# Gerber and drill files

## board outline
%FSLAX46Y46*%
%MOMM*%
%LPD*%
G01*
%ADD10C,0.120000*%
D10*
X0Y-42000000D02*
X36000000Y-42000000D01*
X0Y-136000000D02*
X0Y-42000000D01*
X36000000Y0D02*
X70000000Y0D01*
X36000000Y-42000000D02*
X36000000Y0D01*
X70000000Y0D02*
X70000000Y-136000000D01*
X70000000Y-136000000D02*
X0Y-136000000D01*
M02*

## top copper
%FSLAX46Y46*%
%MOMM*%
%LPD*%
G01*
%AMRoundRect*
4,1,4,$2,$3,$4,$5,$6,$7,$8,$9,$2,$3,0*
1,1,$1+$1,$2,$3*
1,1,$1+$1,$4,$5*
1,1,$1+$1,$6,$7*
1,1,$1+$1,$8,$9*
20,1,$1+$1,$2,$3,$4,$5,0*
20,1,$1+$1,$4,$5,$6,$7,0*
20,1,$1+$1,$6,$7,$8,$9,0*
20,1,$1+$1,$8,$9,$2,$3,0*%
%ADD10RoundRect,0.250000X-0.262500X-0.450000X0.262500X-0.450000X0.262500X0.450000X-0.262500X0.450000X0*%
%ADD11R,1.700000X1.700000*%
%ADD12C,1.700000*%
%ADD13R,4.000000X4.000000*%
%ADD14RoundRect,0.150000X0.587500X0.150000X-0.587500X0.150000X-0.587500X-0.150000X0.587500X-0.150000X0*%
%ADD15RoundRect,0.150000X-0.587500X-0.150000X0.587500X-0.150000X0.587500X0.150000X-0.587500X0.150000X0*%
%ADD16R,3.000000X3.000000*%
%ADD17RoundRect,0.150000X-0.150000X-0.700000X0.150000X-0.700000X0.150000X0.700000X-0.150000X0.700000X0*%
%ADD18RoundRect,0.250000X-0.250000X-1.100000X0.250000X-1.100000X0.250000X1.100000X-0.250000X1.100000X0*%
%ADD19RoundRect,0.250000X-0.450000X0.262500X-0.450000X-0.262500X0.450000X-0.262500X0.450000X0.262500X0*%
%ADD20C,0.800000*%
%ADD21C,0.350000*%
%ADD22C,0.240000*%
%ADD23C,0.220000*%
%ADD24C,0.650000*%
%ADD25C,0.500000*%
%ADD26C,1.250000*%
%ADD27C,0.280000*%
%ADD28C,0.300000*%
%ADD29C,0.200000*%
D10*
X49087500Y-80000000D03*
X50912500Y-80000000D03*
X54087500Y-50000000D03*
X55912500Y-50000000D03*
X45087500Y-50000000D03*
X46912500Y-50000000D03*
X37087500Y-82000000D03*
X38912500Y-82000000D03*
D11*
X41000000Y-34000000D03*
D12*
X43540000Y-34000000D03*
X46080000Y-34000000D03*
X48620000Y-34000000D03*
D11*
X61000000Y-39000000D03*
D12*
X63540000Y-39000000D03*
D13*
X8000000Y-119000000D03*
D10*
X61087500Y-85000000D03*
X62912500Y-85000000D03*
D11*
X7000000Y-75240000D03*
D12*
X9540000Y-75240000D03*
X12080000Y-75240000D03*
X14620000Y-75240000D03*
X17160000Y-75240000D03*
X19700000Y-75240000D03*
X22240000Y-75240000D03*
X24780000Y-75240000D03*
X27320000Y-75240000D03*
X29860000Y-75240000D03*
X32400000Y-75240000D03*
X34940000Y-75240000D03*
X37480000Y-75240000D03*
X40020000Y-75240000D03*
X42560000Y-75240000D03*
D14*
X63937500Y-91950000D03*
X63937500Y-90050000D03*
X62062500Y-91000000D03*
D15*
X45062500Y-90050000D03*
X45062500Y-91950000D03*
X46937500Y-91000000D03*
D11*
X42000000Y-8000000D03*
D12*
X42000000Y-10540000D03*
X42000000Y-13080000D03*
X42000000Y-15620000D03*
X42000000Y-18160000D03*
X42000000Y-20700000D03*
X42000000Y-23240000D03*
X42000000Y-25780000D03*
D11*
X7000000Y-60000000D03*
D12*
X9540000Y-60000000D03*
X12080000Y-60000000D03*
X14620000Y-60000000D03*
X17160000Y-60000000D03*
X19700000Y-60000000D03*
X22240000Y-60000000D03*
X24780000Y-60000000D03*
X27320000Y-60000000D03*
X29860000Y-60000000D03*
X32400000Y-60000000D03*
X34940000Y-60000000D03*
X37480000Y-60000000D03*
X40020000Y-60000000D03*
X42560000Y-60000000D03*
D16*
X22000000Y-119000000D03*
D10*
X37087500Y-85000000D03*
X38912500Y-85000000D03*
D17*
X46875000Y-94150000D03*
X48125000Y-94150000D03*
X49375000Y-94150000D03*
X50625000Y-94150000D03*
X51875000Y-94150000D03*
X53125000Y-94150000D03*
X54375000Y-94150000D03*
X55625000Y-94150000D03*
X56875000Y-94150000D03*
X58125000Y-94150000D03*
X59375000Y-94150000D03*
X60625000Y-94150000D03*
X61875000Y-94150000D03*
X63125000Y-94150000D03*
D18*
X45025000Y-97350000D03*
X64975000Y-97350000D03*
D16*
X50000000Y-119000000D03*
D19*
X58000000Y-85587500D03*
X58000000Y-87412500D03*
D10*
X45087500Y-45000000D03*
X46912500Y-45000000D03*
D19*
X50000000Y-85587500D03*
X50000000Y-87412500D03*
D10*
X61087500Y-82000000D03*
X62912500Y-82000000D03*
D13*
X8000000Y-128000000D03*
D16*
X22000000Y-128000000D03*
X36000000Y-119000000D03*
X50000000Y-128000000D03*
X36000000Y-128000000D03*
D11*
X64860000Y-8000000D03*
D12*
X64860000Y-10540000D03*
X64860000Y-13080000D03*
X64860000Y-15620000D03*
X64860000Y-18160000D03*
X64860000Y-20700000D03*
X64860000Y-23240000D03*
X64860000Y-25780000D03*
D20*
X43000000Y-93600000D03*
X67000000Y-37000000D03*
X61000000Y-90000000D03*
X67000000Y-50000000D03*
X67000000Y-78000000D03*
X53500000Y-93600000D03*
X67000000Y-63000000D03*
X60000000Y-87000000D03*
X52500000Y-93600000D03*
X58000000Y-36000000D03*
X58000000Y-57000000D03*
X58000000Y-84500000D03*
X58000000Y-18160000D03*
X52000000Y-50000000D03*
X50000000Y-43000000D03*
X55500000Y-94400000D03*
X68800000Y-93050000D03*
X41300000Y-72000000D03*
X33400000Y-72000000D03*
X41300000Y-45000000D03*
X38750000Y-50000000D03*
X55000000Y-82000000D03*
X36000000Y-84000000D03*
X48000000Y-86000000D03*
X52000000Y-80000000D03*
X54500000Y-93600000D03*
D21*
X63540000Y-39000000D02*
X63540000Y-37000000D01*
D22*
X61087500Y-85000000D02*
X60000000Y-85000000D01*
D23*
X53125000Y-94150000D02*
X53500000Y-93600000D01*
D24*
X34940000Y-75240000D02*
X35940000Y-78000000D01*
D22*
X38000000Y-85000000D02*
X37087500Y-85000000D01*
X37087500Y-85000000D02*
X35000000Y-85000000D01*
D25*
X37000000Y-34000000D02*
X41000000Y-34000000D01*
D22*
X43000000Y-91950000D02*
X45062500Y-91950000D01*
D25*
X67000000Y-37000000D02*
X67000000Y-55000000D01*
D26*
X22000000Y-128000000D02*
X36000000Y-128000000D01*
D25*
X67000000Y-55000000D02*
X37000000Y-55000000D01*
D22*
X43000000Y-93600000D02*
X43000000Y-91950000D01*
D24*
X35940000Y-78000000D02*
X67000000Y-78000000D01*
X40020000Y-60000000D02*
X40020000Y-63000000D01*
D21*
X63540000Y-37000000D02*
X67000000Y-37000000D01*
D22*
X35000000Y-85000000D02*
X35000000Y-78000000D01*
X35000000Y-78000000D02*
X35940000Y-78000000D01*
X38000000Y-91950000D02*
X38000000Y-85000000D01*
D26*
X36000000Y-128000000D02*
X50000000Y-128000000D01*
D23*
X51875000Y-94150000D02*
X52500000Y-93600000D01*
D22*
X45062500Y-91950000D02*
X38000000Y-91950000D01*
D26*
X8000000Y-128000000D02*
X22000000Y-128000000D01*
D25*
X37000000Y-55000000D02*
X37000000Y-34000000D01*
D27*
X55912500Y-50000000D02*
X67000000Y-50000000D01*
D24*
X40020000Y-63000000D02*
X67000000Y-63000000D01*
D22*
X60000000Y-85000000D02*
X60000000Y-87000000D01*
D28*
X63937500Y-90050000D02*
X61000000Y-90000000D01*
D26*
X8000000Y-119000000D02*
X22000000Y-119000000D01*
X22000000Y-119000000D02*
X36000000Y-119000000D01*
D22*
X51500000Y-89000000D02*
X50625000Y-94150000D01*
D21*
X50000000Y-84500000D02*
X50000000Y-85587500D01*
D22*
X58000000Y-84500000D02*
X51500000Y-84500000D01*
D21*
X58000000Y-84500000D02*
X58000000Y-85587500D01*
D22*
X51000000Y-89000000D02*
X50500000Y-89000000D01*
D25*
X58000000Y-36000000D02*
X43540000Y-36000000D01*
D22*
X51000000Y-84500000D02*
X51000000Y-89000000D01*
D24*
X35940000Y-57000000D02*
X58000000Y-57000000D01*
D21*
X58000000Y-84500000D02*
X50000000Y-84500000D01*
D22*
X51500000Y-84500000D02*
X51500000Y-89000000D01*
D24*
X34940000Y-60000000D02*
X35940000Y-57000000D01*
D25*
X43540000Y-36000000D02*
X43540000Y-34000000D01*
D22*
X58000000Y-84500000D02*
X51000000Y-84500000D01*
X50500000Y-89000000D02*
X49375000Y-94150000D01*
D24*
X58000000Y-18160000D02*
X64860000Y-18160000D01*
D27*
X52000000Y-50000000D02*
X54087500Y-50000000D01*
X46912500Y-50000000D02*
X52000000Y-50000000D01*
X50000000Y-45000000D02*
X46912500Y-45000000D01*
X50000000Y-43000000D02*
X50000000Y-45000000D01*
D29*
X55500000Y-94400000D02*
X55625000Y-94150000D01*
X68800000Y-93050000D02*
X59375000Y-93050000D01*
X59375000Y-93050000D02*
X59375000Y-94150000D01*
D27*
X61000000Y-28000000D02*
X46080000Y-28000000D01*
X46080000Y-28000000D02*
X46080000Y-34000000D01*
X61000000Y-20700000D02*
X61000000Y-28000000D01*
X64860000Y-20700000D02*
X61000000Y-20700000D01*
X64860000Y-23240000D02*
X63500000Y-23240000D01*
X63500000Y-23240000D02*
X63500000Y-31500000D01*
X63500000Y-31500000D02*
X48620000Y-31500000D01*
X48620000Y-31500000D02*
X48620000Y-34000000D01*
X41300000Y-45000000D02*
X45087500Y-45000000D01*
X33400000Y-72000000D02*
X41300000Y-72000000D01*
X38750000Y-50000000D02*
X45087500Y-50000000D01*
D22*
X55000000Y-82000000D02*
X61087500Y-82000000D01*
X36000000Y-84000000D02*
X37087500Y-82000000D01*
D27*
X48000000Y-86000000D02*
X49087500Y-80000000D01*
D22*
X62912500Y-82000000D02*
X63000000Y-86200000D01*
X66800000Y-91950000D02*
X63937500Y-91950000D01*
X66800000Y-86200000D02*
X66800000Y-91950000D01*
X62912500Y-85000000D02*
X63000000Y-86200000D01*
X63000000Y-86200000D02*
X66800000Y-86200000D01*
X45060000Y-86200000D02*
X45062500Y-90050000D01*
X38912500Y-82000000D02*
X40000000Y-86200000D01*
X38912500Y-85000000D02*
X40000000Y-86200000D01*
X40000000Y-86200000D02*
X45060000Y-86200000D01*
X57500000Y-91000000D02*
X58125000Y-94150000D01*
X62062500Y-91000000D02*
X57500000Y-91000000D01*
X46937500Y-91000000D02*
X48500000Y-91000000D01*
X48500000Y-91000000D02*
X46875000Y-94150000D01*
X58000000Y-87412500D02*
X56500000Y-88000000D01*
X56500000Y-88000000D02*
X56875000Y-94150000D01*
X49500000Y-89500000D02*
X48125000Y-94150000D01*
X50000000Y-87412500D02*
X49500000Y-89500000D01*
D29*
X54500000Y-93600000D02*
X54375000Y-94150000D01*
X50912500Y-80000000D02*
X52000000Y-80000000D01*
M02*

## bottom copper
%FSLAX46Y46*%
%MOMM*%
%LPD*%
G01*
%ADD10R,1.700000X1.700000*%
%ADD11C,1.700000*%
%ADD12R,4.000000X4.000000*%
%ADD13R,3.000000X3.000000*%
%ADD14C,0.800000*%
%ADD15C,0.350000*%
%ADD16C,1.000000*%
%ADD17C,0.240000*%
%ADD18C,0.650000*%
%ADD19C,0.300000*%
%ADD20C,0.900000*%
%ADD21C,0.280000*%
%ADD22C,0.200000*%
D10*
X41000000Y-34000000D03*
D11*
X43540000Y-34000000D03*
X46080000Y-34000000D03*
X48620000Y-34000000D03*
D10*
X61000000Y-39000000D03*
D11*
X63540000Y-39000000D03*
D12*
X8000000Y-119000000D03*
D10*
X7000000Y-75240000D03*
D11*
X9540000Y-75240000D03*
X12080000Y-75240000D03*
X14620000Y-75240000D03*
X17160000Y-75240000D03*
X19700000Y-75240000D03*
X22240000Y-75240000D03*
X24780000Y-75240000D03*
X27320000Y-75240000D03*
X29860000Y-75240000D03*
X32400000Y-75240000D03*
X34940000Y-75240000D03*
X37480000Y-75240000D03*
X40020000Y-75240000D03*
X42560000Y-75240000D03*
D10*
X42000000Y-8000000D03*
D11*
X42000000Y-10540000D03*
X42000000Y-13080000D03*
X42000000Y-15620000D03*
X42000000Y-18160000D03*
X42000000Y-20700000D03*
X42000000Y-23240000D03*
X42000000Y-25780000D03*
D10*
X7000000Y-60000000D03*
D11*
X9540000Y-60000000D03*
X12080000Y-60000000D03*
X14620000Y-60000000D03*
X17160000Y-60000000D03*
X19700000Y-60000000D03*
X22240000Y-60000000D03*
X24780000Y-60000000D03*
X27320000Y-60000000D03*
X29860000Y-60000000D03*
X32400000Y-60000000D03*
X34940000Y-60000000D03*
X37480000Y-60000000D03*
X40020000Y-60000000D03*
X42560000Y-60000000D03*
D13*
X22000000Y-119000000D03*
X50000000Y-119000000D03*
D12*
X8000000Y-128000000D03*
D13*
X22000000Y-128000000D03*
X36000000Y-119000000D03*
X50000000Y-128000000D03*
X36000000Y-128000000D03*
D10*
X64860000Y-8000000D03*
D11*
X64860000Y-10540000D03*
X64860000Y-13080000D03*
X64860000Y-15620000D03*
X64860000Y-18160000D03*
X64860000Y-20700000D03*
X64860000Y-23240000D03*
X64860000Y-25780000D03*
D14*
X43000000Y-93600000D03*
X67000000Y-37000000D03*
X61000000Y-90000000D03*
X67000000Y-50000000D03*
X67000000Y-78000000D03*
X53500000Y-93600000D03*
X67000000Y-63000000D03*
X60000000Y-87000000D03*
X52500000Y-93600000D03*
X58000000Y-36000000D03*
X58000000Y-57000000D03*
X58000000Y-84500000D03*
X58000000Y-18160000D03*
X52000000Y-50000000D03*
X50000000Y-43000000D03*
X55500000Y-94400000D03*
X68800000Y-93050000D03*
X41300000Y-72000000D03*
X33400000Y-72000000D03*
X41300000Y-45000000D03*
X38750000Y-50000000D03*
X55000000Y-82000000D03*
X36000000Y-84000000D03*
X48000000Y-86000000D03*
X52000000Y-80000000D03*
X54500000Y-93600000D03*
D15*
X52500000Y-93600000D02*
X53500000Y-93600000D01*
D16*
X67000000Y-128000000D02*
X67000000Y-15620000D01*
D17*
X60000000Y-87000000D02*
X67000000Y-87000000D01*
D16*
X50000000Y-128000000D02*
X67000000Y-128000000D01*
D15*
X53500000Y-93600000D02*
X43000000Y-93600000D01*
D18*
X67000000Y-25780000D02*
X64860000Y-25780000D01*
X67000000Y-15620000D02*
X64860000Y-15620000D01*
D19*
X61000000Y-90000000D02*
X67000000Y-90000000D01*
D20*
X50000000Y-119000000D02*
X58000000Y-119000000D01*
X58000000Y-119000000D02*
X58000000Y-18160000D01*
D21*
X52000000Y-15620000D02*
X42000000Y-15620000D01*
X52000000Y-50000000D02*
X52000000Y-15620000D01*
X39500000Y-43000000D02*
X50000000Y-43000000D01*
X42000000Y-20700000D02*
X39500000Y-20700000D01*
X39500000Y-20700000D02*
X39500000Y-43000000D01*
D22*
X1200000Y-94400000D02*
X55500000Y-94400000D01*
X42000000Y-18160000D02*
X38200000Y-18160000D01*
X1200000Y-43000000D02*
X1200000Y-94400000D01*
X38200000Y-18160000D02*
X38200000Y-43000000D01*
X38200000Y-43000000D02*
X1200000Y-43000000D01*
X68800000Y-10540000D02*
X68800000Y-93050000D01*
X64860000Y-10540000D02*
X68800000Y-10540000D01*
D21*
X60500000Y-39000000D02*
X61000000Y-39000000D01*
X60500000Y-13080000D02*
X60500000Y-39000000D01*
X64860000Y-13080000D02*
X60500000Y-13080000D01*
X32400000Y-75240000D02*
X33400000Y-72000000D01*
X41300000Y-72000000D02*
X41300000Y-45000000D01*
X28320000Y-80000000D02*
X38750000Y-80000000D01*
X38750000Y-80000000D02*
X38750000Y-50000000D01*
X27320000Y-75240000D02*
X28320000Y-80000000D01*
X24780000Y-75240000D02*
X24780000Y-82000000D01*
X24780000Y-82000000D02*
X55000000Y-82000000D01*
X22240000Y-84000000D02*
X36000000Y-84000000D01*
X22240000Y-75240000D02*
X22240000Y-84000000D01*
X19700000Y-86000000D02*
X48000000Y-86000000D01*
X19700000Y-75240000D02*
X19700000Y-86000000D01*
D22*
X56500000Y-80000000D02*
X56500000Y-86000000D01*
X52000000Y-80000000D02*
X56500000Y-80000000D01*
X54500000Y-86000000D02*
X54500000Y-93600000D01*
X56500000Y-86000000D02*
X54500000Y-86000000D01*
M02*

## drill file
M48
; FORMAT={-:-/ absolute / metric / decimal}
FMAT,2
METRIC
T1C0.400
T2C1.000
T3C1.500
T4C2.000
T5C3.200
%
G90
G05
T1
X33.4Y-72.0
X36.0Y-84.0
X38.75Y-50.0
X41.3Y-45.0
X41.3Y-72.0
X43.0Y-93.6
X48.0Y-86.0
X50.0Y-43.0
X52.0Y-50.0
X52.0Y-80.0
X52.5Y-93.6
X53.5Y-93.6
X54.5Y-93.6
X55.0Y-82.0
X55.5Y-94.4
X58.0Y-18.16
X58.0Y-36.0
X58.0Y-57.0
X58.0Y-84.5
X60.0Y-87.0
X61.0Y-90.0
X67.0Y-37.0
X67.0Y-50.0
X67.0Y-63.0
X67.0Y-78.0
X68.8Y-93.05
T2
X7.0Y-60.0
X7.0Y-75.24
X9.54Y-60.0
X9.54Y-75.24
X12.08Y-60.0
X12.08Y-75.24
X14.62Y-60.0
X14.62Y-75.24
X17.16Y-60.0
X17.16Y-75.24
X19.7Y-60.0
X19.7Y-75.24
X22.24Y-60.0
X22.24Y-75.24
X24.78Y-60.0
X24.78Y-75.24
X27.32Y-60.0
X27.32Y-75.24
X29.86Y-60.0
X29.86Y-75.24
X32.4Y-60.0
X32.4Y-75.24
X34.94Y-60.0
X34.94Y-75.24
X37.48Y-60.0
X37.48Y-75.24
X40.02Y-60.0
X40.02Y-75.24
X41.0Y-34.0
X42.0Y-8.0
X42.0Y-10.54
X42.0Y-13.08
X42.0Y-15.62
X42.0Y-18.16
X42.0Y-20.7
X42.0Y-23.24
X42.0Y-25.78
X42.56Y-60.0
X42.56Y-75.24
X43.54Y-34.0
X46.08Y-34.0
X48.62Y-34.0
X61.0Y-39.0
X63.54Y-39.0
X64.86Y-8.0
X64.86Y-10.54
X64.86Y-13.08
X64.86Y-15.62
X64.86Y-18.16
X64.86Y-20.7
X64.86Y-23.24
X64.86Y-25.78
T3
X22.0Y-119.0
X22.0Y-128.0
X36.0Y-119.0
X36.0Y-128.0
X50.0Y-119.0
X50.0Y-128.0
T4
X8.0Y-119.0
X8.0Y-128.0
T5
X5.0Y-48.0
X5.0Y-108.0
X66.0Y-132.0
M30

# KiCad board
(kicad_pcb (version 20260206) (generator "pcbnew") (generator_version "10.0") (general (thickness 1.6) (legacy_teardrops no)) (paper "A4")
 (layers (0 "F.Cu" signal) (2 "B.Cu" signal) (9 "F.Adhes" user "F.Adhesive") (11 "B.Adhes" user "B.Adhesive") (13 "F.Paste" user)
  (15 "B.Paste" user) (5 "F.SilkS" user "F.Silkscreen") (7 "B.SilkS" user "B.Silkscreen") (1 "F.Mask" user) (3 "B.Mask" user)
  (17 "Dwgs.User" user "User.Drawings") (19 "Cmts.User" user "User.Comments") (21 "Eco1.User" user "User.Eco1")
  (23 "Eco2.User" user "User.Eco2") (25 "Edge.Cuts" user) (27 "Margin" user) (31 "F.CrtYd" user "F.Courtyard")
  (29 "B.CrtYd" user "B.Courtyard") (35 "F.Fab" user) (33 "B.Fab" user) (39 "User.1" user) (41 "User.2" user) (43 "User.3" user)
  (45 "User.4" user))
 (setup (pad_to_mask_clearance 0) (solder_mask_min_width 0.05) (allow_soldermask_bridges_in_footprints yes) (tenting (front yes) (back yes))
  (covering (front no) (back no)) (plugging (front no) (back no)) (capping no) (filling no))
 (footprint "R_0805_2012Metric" (layer "F.Cu") (at 50 80)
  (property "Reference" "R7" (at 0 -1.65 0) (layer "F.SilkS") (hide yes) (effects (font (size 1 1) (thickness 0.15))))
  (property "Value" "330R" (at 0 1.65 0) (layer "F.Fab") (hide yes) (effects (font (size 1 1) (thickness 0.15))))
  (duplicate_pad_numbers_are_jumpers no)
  (pad "1" smd roundrect (at -0.9125 0) (size 1.025 1.4) (layers "F.Cu" "F.Mask" "F.Paste") (roundrect_rratio 0.243902)
   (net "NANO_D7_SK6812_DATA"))
  (pad "2" smd roundrect (at 0.9125 0) (size 1.025 1.4) (layers "F.Cu" "F.Mask" "F.Paste") (roundrect_rratio 0.243902) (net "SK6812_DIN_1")))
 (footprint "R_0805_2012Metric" (layer "F.Cu") (at 55 50)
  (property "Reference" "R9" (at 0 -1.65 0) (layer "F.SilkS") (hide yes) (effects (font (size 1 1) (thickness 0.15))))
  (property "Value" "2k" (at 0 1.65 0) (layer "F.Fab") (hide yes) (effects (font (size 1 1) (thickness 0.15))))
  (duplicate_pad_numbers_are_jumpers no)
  (pad "1" smd roundrect (at -0.9125 0) (size 1.025 1.4) (layers "F.Cu" "F.Mask" "F.Paste") (roundrect_rratio 0.243902)
   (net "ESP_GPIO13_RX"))
  (pad "2" smd roundrect (at 0.9125 0) (size 1.025 1.4) (layers "F.Cu" "F.Mask" "F.Paste") (roundrect_rratio 0.243902) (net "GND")))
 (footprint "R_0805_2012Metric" (layer "F.Cu") (at 46 50)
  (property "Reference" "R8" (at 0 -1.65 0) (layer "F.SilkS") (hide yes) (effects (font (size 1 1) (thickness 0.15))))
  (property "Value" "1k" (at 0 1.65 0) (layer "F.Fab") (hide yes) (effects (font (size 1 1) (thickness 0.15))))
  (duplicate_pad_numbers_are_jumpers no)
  (pad "1" smd roundrect (at -0.9125 0) (size 1.025 1.4) (layers "F.Cu" "F.Mask" "F.Paste") (roundrect_rratio 0.243902) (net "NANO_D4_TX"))
  (pad "2" smd roundrect (at 0.9125 0) (size 1.025 1.4) (layers "F.Cu" "F.Mask" "F.Paste") (roundrect_rratio 0.243902) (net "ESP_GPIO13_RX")))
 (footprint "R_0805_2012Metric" (layer "F.Cu") (at 38 82)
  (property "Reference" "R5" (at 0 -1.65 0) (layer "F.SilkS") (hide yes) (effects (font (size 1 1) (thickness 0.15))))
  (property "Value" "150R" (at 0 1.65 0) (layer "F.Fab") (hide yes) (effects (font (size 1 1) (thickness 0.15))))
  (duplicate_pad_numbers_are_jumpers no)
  (pad "1" smd roundrect (at -0.9125 0) (size 1.025 1.4) (layers "F.Cu" "F.Mask" "F.Paste") (roundrect_rratio 0.243902)
   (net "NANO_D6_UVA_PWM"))
  (pad "2" smd roundrect (at 0.9125 0) (size 1.025 1.4) (layers "F.Cu" "F.Mask" "F.Paste") (roundrect_rratio 0.243902) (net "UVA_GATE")))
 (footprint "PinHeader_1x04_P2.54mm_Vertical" (layer "F.Cu") (at 41 34 90)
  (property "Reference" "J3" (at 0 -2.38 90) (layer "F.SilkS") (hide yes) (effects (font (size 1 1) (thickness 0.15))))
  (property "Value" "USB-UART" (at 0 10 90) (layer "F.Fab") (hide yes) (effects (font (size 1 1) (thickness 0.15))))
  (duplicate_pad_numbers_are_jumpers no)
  (pad "1" thru_hole rect (at 0 0 90) (size 1.7 1.7) (drill 1) (layers "*.Cu" "*.Mask") (remove_unused_layers no) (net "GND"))
  (pad "2" thru_hole circle (at 0 2.54 90) (size 1.7 1.7) (drill 1) (layers "*.Cu" "*.Mask") (remove_unused_layers no) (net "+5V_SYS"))
  (pad "3" thru_hole circle (at 0 5.08 90) (size 1.7 1.7) (drill 1) (layers "*.Cu" "*.Mask") (remove_unused_layers no) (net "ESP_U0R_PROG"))
  (pad "4" thru_hole circle (at 0 7.62 90) (size 1.7 1.7) (drill 1) (layers "*.Cu" "*.Mask") (remove_unused_layers no) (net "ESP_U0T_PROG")))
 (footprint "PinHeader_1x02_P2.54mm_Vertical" (layer "F.Cu") (at 61 39 90)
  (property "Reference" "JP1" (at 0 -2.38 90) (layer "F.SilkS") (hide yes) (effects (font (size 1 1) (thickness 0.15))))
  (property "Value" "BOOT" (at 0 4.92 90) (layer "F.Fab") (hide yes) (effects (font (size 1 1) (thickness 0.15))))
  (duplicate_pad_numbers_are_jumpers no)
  (pad "1" thru_hole rect (at 0 0 90) (size 1.7 1.7) (drill 1) (layers "*.Cu" "*.Mask") (remove_unused_layers no) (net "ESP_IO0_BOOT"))
  (pad "2" thru_hole circle (at 0 2.54 90) (size 1.7 1.7) (drill 1) (layers "*.Cu" "*.Mask") (remove_unused_layers no) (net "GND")))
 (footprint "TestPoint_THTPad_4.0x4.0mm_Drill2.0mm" (layer "F.Cu") (at 8 119)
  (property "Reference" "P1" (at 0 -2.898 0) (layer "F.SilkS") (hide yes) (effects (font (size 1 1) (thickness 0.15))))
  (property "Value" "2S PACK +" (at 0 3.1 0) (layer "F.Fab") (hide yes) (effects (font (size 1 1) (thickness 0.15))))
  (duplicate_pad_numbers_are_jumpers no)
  (pad "1" thru_hole rect (at 0 0) (size 4 4) (drill 2) (layers "*.Cu" "*.Mask") (remove_unused_layers no) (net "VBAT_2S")))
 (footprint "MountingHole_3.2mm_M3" (layer "F.Cu") (at 5 48)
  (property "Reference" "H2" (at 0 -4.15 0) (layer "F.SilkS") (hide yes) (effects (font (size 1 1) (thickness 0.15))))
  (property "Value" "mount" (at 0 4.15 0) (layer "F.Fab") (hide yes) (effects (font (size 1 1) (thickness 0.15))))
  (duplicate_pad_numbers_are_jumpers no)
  (pad "" np_thru_hole circle (at 0 0) (size 3.2 3.2) (drill 3.2) (layers "*.Cu" "*.Mask")))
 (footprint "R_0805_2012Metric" (layer "F.Cu") (at 62 85)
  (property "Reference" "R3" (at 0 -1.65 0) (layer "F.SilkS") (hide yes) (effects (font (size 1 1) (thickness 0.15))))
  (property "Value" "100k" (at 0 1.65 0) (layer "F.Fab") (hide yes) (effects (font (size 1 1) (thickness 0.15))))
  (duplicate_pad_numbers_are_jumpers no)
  (pad "1" smd roundrect (at -0.9125 0) (size 1.025 1.4) (layers "F.Cu" "F.Mask" "F.Paste") (roundrect_rratio 0.243902) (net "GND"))
  (pad "2" smd roundrect (at 0.9125 0) (size 1.025 1.4) (layers "F.Cu" "F.Mask" "F.Paste") (roundrect_rratio 0.243902) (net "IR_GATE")))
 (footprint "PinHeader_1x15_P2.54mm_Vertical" (layer "F.Cu") (at 7 75.24 90)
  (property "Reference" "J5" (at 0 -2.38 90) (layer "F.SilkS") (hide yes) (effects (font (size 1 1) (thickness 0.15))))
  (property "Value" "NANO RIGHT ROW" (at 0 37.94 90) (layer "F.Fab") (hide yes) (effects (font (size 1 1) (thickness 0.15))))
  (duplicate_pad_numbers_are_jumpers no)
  (pad "1" thru_hole rect (at 0 0 90) (size 1.7 1.7) (drill 1) (layers "*.Cu" "*.Mask") (remove_unused_layers no))
  (pad "2" thru_hole circle (at 0 2.54 90) (size 1.7 1.7) (drill 1) (layers "*.Cu" "*.Mask") (remove_unused_layers no))
  (pad "3" thru_hole circle (at 0 5.08 90) (size 1.7 1.7) (drill 1) (layers "*.Cu" "*.Mask") (remove_unused_layers no))
  (pad "4" thru_hole circle (at 0 7.62 90) (size 1.7 1.7) (drill 1) (layers "*.Cu" "*.Mask") (remove_unused_layers no))
  (pad "5" thru_hole circle (at 0 10.16 90) (size 1.7 1.7) (drill 1) (layers "*.Cu" "*.Mask") (remove_unused_layers no)
   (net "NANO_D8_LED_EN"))
  (pad "6" thru_hole circle (at 0 12.7 90) (size 1.7 1.7) (drill 1) (layers "*.Cu" "*.Mask") (remove_unused_layers no)
   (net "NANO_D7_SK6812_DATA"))
  (pad "7" thru_hole circle (at 0 15.24 90) (size 1.7 1.7) (drill 1) (layers "*.Cu" "*.Mask") (remove_unused_layers no)
   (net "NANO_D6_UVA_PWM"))
  (pad "8" thru_hole circle (at 0 17.78 90) (size 1.7 1.7) (drill 1) (layers "*.Cu" "*.Mask") (remove_unused_layers no)
   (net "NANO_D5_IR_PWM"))
  (pad "9" thru_hole circle (at 0 20.32 90) (size 1.7 1.7) (drill 1) (layers "*.Cu" "*.Mask") (remove_unused_layers no) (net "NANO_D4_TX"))
  (pad "10" thru_hole circle (at 0 22.86 90) (size 1.7 1.7) (drill 1) (layers "*.Cu" "*.Mask") (remove_unused_layers no))
  (pad "11" thru_hole circle (at 0 25.4 90) (size 1.7 1.7) (drill 1) (layers "*.Cu" "*.Mask") (remove_unused_layers no) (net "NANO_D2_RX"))
  (pad "12" thru_hole circle (at 0 27.94 90) (size 1.7 1.7) (drill 1) (layers "*.Cu" "*.Mask") (remove_unused_layers no) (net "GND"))
  (pad "13" thru_hole circle (at 0 30.48 90) (size 1.7 1.7) (drill 1) (layers "*.Cu" "*.Mask") (remove_unused_layers no))
  (pad "14" thru_hole circle (at 0 33.02 90) (size 1.7 1.7) (drill 1) (layers "*.Cu" "*.Mask") (remove_unused_layers no))
  (pad "15" thru_hole circle (at 0 35.56 90) (size 1.7 1.7) (drill 1) (layers "*.Cu" "*.Mask") (remove_unused_layers no)))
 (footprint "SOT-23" (layer "F.Cu") (at 63 91 180)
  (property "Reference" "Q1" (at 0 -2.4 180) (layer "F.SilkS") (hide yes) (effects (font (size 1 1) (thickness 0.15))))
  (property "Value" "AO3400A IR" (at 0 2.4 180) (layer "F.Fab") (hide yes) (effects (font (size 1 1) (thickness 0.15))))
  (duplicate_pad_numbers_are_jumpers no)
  (pad "1" smd roundrect (at -0.9375 -0.95 180) (size 1.475 0.6) (layers "F.Cu" "F.Mask" "F.Paste") (roundrect_rratio 0.25) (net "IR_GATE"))
  (pad "2" smd roundrect (at -0.9375 0.95 180) (size 1.475 0.6) (layers "F.Cu" "F.Mask" "F.Paste") (roundrect_rratio 0.25) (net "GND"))
  (pad "3" smd roundrect (at 0.9375 0 180) (size 1.475 0.6) (layers "F.Cu" "F.Mask" "F.Paste") (roundrect_rratio 0.25) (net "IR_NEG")))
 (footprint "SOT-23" (layer "F.Cu") (at 46 91)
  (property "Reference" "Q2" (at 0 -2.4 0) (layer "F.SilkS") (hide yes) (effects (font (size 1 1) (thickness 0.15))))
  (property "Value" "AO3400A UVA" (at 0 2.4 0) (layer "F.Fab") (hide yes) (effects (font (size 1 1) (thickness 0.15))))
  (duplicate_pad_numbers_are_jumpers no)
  (pad "1" smd roundrect (at -0.9375 -0.95) (size 1.475 0.6) (layers "F.Cu" "F.Mask" "F.Paste") (roundrect_rratio 0.25) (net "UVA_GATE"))
  (pad "2" smd roundrect (at -0.9375 0.95) (size 1.475 0.6) (layers "F.Cu" "F.Mask" "F.Paste") (roundrect_rratio 0.25) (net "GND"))
  (pad "3" smd roundrect (at 0.9375 0) (size 1.475 0.6) (layers "F.Cu" "F.Mask" "F.Paste") (roundrect_rratio 0.25) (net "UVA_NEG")))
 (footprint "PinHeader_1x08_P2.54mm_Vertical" (layer "F.Cu") (at 42 8)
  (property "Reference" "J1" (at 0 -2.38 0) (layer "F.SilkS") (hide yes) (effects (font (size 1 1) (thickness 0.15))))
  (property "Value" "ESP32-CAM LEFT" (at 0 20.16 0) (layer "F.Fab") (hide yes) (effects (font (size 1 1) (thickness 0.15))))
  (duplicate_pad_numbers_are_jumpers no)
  (pad "1" thru_hole rect (at 0 0) (size 1.7 1.7) (drill 1) (layers "*.Cu" "*.Mask") (remove_unused_layers no))
  (pad "2" thru_hole circle (at 0 2.54) (size 1.7 1.7) (drill 1) (layers "*.Cu" "*.Mask") (remove_unused_layers no))
  (pad "3" thru_hole circle (at 0 5.08) (size 1.7 1.7) (drill 1) (layers "*.Cu" "*.Mask") (remove_unused_layers no))
  (pad "4" thru_hole circle (at 0 7.62) (size 1.7 1.7) (drill 1) (layers "*.Cu" "*.Mask") (remove_unused_layers no) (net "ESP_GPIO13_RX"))
  (pad "5" thru_hole circle (at 0 10.16) (size 1.7 1.7) (drill 1) (layers "*.Cu" "*.Mask") (remove_unused_layers no)
   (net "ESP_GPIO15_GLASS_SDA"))
  (pad "6" thru_hole circle (at 0 12.7) (size 1.7 1.7) (drill 1) (layers "*.Cu" "*.Mask") (remove_unused_layers no) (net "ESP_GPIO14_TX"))
  (pad "7" thru_hole circle (at 0 15.24) (size 1.7 1.7) (drill 1) (layers "*.Cu" "*.Mask") (remove_unused_layers no))
  (pad "8" thru_hole circle (at 0 17.78) (size 1.7 1.7) (drill 1) (layers "*.Cu" "*.Mask") (remove_unused_layers no)))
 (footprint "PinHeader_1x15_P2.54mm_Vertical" (layer "F.Cu") (at 7 60 90)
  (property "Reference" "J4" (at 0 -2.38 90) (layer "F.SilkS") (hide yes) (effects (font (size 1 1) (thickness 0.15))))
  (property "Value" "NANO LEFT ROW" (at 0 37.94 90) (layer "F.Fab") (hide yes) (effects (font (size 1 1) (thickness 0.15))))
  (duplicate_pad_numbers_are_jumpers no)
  (pad "1" thru_hole rect (at 0 0 90) (size 1.7 1.7) (drill 1) (layers "*.Cu" "*.Mask") (remove_unused_layers no))
  (pad "2" thru_hole circle (at 0 2.54 90) (size 1.7 1.7) (drill 1) (layers "*.Cu" "*.Mask") (remove_unused_layers no))
  (pad "3" thru_hole circle (at 0 5.08 90) (size 1.7 1.7) (drill 1) (layers "*.Cu" "*.Mask") (remove_unused_layers no))
  (pad "4" thru_hole circle (at 0 7.62 90) (size 1.7 1.7) (drill 1) (layers "*.Cu" "*.Mask") (remove_unused_layers no))
  (pad "5" thru_hole circle (at 0 10.16 90) (size 1.7 1.7) (drill 1) (layers "*.Cu" "*.Mask") (remove_unused_layers no))
  (pad "6" thru_hole circle (at 0 12.7 90) (size 1.7 1.7) (drill 1) (layers "*.Cu" "*.Mask") (remove_unused_layers no))
  (pad "7" thru_hole circle (at 0 15.24 90) (size 1.7 1.7) (drill 1) (layers "*.Cu" "*.Mask") (remove_unused_layers no))
  (pad "8" thru_hole circle (at 0 17.78 90) (size 1.7 1.7) (drill 1) (layers "*.Cu" "*.Mask") (remove_unused_layers no))
  (pad "9" thru_hole circle (at 0 20.32 90) (size 1.7 1.7) (drill 1) (layers "*.Cu" "*.Mask") (remove_unused_layers no))
  (pad "10" thru_hole circle (at 0 22.86 90) (size 1.7 1.7) (drill 1) (layers "*.Cu" "*.Mask") (remove_unused_layers no))
  (pad "11" thru_hole circle (at 0 25.4 90) (size 1.7 1.7) (drill 1) (layers "*.Cu" "*.Mask") (remove_unused_layers no))
  (pad "12" thru_hole circle (at 0 27.94 90) (size 1.7 1.7) (drill 1) (layers "*.Cu" "*.Mask") (remove_unused_layers no) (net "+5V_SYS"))
  (pad "13" thru_hole circle (at 0 30.48 90) (size 1.7 1.7) (drill 1) (layers "*.Cu" "*.Mask") (remove_unused_layers no))
  (pad "14" thru_hole circle (at 0 33.02 90) (size 1.7 1.7) (drill 1) (layers "*.Cu" "*.Mask") (remove_unused_layers no) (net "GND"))
  (pad "15" thru_hole circle (at 0 35.56 90) (size 1.7 1.7) (drill 1) (layers "*.Cu" "*.Mask") (remove_unused_layers no)))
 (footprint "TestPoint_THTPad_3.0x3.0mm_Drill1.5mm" (layer "F.Cu") (at 22 119)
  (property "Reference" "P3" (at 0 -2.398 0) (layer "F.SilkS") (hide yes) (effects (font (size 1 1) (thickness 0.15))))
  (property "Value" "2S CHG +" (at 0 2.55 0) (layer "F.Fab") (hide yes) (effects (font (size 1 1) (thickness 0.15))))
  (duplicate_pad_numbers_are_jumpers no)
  (pad "1" thru_hole rect (at 0 0) (size 3 3) (drill 1.5) (layers "*.Cu" "*.Mask") (remove_unused_layers no) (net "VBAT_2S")))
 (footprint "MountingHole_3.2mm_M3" (layer "F.Cu") (at 5 108)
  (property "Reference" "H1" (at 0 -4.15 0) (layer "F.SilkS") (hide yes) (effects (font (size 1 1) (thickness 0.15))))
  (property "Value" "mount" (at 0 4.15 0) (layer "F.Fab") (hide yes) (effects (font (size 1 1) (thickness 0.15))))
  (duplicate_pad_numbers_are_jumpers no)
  (pad "" np_thru_hole circle (at 0 0) (size 3.2 3.2) (drill 3.2) (layers "*.Cu" "*.Mask")))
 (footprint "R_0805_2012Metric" (layer "F.Cu") (at 38 85)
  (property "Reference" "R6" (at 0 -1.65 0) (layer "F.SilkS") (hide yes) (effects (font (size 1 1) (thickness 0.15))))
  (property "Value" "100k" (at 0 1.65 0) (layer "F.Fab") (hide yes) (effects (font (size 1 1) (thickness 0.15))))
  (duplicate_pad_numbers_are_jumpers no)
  (pad "1" smd roundrect (at -0.9125 0) (size 1.025 1.4) (layers "F.Cu" "F.Mask" "F.Paste") (roundrect_rratio 0.243902) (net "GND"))
  (pad "2" smd roundrect (at 0.9125 0) (size 1.025 1.4) (layers "F.Cu" "F.Mask" "F.Paste") (roundrect_rratio 0.243902) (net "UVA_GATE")))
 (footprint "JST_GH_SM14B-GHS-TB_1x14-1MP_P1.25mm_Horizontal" (layer "F.Cu") (at 55 96)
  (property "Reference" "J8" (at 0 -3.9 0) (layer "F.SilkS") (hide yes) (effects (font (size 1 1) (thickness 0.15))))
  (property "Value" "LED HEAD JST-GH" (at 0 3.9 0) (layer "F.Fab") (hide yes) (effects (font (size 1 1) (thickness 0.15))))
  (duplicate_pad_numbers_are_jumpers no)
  (pad "1" smd roundrect (at -8.125 -1.85) (size 0.6 1.7) (layers "F.Cu" "F.Mask" "F.Paste") (roundrect_rratio 0.25) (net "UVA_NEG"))
  (pad "2" smd roundrect (at -6.875 -1.85) (size 0.6 1.7) (layers "F.Cu" "F.Mask" "F.Paste") (roundrect_rratio 0.25) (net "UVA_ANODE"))
  (pad "3" smd roundrect (at -5.625 -1.85) (size 0.6 1.7) (layers "F.Cu" "F.Mask" "F.Paste") (roundrect_rratio 0.25) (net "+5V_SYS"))
  (pad "4" smd roundrect (at -4.375 -1.85) (size 0.6 1.7) (layers "F.Cu" "F.Mask" "F.Paste") (roundrect_rratio 0.25) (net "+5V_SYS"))
  (pad "5" smd roundrect (at -3.125 -1.85) (size 0.6 1.7) (layers "F.Cu" "F.Mask" "F.Paste") (roundrect_rratio 0.25) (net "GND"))
  (pad "6" smd roundrect (at -1.875 -1.85) (size 0.6 1.7) (layers "F.Cu" "F.Mask" "F.Paste") (roundrect_rratio 0.25) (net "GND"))
  (pad "7" smd roundrect (at -0.625 -1.85) (size 0.6 1.7) (layers "F.Cu" "F.Mask" "F.Paste") (roundrect_rratio 0.25) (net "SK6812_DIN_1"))
  (pad "8" smd roundrect (at 0.625 -1.85) (size 0.6 1.7) (layers "F.Cu" "F.Mask" "F.Paste") (roundrect_rratio 0.25)
   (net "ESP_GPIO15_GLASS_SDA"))
  (pad "9" smd roundrect (at 1.875 -1.85) (size 0.6 1.7) (layers "F.Cu" "F.Mask" "F.Paste") (roundrect_rratio 0.25) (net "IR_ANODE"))
  (pad "10" smd roundrect (at 3.125 -1.85) (size 0.6 1.7) (layers "F.Cu" "F.Mask" "F.Paste") (roundrect_rratio 0.25) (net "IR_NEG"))
  (pad "11" smd roundrect (at 4.375 -1.85) (size 0.6 1.7) (layers "F.Cu" "F.Mask" "F.Paste") (roundrect_rratio 0.25)
   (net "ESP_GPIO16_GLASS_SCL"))
  (pad "12" smd roundrect (at 5.625 -1.85) (size 0.6 1.7) (layers "F.Cu" "F.Mask" "F.Paste") (roundrect_rratio 0.25))
  (pad "13" smd roundrect (at 6.875 -1.85) (size 0.6 1.7) (layers "F.Cu" "F.Mask" "F.Paste") (roundrect_rratio 0.25))
  (pad "14" smd roundrect (at 8.125 -1.85) (size 0.6 1.7) (layers "F.Cu" "F.Mask" "F.Paste") (roundrect_rratio 0.25))
  (pad "MP" smd roundrect (at -9.975 1.35) (size 1 2.7) (layers "F.Cu" "F.Mask" "F.Paste") (roundrect_rratio 0.25))
  (pad "MP" smd roundrect (at 9.975 1.35) (size 1 2.7) (layers "F.Cu" "F.Mask" "F.Paste") (roundrect_rratio 0.25)))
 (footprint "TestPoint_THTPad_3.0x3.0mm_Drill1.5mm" (layer "F.Cu") (at 50 119)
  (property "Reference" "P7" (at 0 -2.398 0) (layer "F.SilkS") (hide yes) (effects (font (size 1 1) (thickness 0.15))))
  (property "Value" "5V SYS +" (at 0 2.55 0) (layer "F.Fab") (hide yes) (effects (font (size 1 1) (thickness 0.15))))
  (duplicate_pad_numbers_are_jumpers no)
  (pad "1" thru_hole rect (at 0 0) (size 3 3) (drill 1.5) (layers "*.Cu" "*.Mask") (remove_unused_layers no) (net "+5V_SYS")))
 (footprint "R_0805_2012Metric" (layer "F.Cu") (at 58 86.5 -90)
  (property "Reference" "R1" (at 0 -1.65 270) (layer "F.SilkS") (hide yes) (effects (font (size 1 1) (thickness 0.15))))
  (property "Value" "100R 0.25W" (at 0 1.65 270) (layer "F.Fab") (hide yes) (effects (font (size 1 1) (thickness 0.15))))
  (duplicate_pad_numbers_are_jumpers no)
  (pad "1" smd roundrect (at -0.9125 0 270) (size 1.025 1.4) (layers "F.Cu" "F.Mask" "F.Paste") (roundrect_rratio 0.243902) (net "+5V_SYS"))
  (pad "2" smd roundrect (at 0.9125 0 270) (size 1.025 1.4) (layers "F.Cu" "F.Mask" "F.Paste") (roundrect_rratio 0.243902) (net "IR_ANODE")))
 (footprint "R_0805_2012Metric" (layer "F.Cu") (at 46 45)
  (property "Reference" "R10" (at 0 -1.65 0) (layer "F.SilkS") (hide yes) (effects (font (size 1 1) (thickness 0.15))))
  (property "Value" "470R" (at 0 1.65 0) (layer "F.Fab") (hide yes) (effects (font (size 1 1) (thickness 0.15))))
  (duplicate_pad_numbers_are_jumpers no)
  (pad "1" smd roundrect (at -0.9125 0) (size 1.025 1.4) (layers "F.Cu" "F.Mask" "F.Paste") (roundrect_rratio 0.243902) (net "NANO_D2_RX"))
  (pad "2" smd roundrect (at 0.9125 0) (size 1.025 1.4) (layers "F.Cu" "F.Mask" "F.Paste") (roundrect_rratio 0.243902) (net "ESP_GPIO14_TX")))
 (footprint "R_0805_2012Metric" (layer "F.Cu") (at 50 86.5 -90)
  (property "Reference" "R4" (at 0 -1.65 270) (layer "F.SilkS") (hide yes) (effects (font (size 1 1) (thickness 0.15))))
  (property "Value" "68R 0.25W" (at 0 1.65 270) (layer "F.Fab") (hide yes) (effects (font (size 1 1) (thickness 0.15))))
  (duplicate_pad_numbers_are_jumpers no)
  (pad "1" smd roundrect (at -0.9125 0 270) (size 1.025 1.4) (layers "F.Cu" "F.Mask" "F.Paste") (roundrect_rratio 0.243902) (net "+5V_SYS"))
  (pad "2" smd roundrect (at 0.9125 0 270) (size 1.025 1.4) (layers "F.Cu" "F.Mask" "F.Paste") (roundrect_rratio 0.243902) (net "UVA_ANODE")))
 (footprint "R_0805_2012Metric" (layer "F.Cu") (at 62 82)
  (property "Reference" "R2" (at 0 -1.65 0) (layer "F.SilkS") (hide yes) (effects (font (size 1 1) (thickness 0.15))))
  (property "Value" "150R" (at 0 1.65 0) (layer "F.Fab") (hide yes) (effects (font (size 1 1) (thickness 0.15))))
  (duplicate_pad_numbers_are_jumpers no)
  (pad "1" smd roundrect (at -0.9125 0) (size 1.025 1.4) (layers "F.Cu" "F.Mask" "F.Paste") (roundrect_rratio 0.243902)
   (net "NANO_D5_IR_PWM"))
  (pad "2" smd roundrect (at 0.9125 0) (size 1.025 1.4) (layers "F.Cu" "F.Mask" "F.Paste") (roundrect_rratio 0.243902) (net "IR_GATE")))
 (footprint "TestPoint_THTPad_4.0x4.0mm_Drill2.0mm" (layer "F.Cu") (at 8 128)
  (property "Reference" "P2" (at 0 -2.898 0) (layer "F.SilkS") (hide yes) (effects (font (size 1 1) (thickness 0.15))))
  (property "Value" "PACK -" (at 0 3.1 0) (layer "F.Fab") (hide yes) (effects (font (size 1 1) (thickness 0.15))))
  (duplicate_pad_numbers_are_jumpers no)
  (pad "1" thru_hole rect (at 0 0) (size 4 4) (drill 2) (layers "*.Cu" "*.Mask") (remove_unused_layers no) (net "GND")))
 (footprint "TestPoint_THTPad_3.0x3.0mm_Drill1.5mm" (layer "F.Cu") (at 22 128)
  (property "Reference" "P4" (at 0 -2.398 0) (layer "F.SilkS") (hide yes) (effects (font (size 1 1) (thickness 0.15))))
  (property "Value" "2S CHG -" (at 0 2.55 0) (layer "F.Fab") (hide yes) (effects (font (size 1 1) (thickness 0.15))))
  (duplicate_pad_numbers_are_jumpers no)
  (pad "1" thru_hole rect (at 0 0) (size 3 3) (drill 1.5) (layers "*.Cu" "*.Mask") (remove_unused_layers no) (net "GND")))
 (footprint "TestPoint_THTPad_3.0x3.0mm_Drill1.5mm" (layer "F.Cu") (at 36 119)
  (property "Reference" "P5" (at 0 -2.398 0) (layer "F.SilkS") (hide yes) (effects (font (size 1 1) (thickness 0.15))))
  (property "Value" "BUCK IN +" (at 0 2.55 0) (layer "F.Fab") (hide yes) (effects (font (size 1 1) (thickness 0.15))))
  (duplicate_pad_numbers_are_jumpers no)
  (pad "1" thru_hole rect (at 0 0) (size 3 3) (drill 1.5) (layers "*.Cu" "*.Mask") (remove_unused_layers no) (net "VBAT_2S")))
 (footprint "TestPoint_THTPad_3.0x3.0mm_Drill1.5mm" (layer "F.Cu") (at 50 128)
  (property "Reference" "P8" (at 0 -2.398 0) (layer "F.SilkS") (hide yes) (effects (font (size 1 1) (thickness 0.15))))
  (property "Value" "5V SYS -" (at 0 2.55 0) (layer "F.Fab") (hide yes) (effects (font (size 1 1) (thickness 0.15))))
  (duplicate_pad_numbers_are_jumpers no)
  (pad "1" thru_hole rect (at 0 0) (size 3 3) (drill 1.5) (layers "*.Cu" "*.Mask") (remove_unused_layers no) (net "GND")))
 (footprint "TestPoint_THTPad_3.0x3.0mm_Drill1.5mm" (layer "F.Cu") (at 36 128)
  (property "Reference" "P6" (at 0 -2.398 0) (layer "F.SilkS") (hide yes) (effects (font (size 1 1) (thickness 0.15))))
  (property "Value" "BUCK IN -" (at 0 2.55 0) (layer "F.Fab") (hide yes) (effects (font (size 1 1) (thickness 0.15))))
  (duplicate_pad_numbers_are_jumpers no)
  (pad "1" thru_hole rect (at 0 0) (size 3 3) (drill 1.5) (layers "*.Cu" "*.Mask") (remove_unused_layers no) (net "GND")))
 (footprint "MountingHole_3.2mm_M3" (layer "F.Cu") (at 66 132)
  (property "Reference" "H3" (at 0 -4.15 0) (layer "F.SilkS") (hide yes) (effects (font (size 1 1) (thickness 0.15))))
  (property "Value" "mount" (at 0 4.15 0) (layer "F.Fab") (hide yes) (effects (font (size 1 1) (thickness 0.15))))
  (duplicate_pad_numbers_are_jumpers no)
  (pad "" np_thru_hole circle (at 0 0) (size 3.2 3.2) (drill 3.2) (layers "*.Cu" "*.Mask")))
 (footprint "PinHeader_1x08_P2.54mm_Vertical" (layer "F.Cu") (at 64.86 8)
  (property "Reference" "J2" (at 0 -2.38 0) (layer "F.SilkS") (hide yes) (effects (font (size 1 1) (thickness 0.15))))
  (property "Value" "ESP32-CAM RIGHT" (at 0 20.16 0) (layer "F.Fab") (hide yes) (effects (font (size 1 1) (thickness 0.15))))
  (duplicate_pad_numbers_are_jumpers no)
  (pad "1" thru_hole rect (at 0 0) (size 1.7 1.7) (drill 1) (layers "*.Cu" "*.Mask") (remove_unused_layers no))
  (pad "2" thru_hole circle (at 0 2.54) (size 1.7 1.7) (drill 1) (layers "*.Cu" "*.Mask") (remove_unused_layers no)
   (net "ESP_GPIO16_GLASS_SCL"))
  (pad "3" thru_hole circle (at 0 5.08) (size 1.7 1.7) (drill 1) (layers "*.Cu" "*.Mask") (remove_unused_layers no) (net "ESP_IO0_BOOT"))
  (pad "4" thru_hole circle (at 0 7.62) (size 1.7 1.7) (drill 1) (layers "*.Cu" "*.Mask") (remove_unused_layers no) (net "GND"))
  (pad "5" thru_hole circle (at 0 10.16) (size 1.7 1.7) (drill 1) (layers "*.Cu" "*.Mask") (remove_unused_layers no) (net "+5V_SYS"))
  (pad "6" thru_hole circle (at 0 12.7) (size 1.7 1.7) (drill 1) (layers "*.Cu" "*.Mask") (remove_unused_layers no) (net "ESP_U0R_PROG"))
  (pad "7" thru_hole circle (at 0 15.24) (size 1.7 1.7) (drill 1) (layers "*.Cu" "*.Mask") (remove_unused_layers no) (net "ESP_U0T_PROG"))
  (pad "8" thru_hole circle (at 0 17.78) (size 1.7 1.7) (drill 1) (layers "*.Cu" "*.Mask") (remove_unused_layers no) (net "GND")))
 (gr_line (start 0 42) (end 36 42) (stroke (width 0.12) (type default)) (layer "Edge.Cuts"))
 (gr_line (start 0 136) (end 0 42) (stroke (width 0.12) (type default)) (layer "Edge.Cuts"))
 (gr_line (start 36 0) (end 70 0) (stroke (width 0.12) (type default)) (layer "Edge.Cuts"))
 (gr_line (start 36 42) (end 36 0) (stroke (width 0.12) (type default)) (layer "Edge.Cuts"))
 (gr_line (start 70 0) (end 70 136) (stroke (width 0.12) (type default)) (layer "Edge.Cuts"))
 (gr_line (start 70 136) (end 0 136) (stroke (width 0.12) (type default)) (layer "Edge.Cuts"))
 (segment (start 63.54 39) (end 63.54 37) (width 0.35) (layer "F.Cu") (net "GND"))
 (segment (start 61.0875 85) (end 60 85) (width 0.24) (layer "F.Cu") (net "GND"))
 (segment (start 53.125 94.15) (end 53.5 93.6) (width 0.22) (layer "F.Cu") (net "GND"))
 (segment (start 34.94 75.24) (end 35.94 78) (width 0.65) (layer "F.Cu") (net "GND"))
 (segment (start 38 85) (end 37.0875 85) (width 0.24) (layer "F.Cu") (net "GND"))
 (segment (start 37.0875 85) (end 35 85) (width 0.24) (layer "F.Cu") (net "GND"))
 (segment (start 37 34) (end 41 34) (width 0.5) (layer "F.Cu") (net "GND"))
 (segment (start 43 91.95) (end 45.0625 91.95) (width 0.24) (layer "F.Cu") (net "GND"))
 (segment (start 67 37) (end 67 55) (width 0.5) (layer "F.Cu") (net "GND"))
 (segment (start 22 128) (end 36 128) (width 1.25) (layer "F.Cu") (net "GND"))
 (segment (start 67 55) (end 37 55) (width 0.5) (layer "F.Cu") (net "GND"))
 (segment (start 43 93.6) (end 43 91.95) (width 0.24) (layer "F.Cu") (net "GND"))
 (segment (start 35.94 78) (end 67 78) (width 0.65) (layer "F.Cu") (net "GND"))
 (segment (start 40.02 60) (end 40.02 63) (width 0.65) (layer "F.Cu") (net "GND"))
 (segment (start 63.54 37) (end 67 37) (width 0.35) (layer "F.Cu") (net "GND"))
 (segment (start 35 85) (end 35 78) (width 0.24) (layer "F.Cu") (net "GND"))
 (segment (start 35 78) (end 35.94 78) (width 0.24) (layer "F.Cu") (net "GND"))
 (segment (start 38 91.95) (end 38 85) (width 0.24) (layer "F.Cu") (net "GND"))
 (segment (start 36 128) (end 50 128) (width 1.25) (layer "F.Cu") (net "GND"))
 (segment (start 51.875 94.15) (end 52.5 93.6) (width 0.22) (layer "F.Cu") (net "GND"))
 (segment (start 45.0625 91.95) (end 38 91.95) (width 0.24) (layer "F.Cu") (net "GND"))
 (segment (start 8 128) (end 22 128) (width 1.25) (layer "F.Cu") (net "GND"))
 (segment (start 37 55) (end 37 34) (width 0.5) (layer "F.Cu") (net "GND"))
 (segment (start 55.9125 50) (end 67 50) (width 0.28) (layer "F.Cu") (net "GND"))
 (segment (start 40.02 63) (end 67 63) (width 0.65) (layer "F.Cu") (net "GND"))
 (segment (start 60 85) (end 60 87) (width 0.24) (layer "F.Cu") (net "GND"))
 (segment (start 63.9375 90.05) (end 61 90) (width 0.3) (layer "F.Cu") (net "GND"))
 (via (at 43 93.6) (size 0.8) (drill 0.4) (layers "F.Cu" "B.Cu") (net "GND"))
 (via (at 67 37) (size 0.8) (drill 0.4) (layers "F.Cu" "B.Cu") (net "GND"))
 (via (at 61 90) (size 0.8) (drill 0.4) (layers "F.Cu" "B.Cu") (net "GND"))
 (via (at 67 50) (size 0.8) (drill 0.4) (layers "F.Cu" "B.Cu") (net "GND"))
 (via (at 67 78) (size 0.8) (drill 0.4) (layers "F.Cu" "B.Cu") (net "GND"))
 (via (at 53.5 93.6) (size 0.8) (drill 0.4) (layers "F.Cu" "B.Cu") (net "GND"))
 (via (at 67 63) (size 0.8) (drill 0.4) (layers "F.Cu" "B.Cu") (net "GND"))
 (via (at 60 87) (size 0.8) (drill 0.4) (layers "F.Cu" "B.Cu") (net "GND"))
 (via (at 52.5 93.6) (size 0.8) (drill 0.4) (layers "F.Cu" "B.Cu") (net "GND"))
 (segment (start 52.5 93.6) (end 53.5 93.6) (width 0.35) (layer "B.Cu") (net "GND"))
 (segment (start 67 128) (end 67 15.62) (width 1) (layer "B.Cu") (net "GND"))
 (segment (start 60 87) (end 67 87) (width 0.24) (layer "B.Cu") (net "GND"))
 (segment (start 50 128) (end 67 128) (width 1) (layer "B.Cu") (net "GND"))
 (segment (start 53.5 93.6) (end 43 93.6) (width 0.35) (layer "B.Cu") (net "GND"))
 (segment (start 67 25.78) (end 64.86 25.78) (width 0.65) (layer "B.Cu") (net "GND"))
 (segment (start 67 15.62) (end 64.86 15.62) (width 0.65) (layer "B.Cu") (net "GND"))
 (segment (start 61 90) (end 67 90) (width 0.3) (layer "B.Cu") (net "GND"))
 (segment (start 8 119) (end 22 119) (width 1.25) (layer "F.Cu") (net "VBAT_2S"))
 (segment (start 22 119) (end 36 119) (width 1.25) (layer "F.Cu") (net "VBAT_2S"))
 (segment (start 51.5 89) (end 50.625 94.15) (width 0.24) (layer "F.Cu") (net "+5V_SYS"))
 (segment (start 50 84.5) (end 50 85.5875) (width 0.35) (layer "F.Cu") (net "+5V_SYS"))
 (segment (start 58 84.5) (end 51.5 84.5) (width 0.24) (layer "F.Cu") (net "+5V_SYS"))
 (segment (start 58 84.5) (end 58 85.5875) (width 0.35) (layer "F.Cu") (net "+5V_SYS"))
 (segment (start 51 89) (end 50.5 89) (width 0.24) (layer "F.Cu") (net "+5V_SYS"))
 (segment (start 58 36) (end 43.54 36) (width 0.5) (layer "F.Cu") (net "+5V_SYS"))
 (segment (start 51 84.5) (end 51 89) (width 0.24) (layer "F.Cu") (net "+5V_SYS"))
 (segment (start 35.94 57) (end 58 57) (width 0.65) (layer "F.Cu") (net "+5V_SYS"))
 (segment (start 58 84.5) (end 50 84.5) (width 0.35) (layer "F.Cu") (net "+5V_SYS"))
 (segment (start 51.5 84.5) (end 51.5 89) (width 0.24) (layer "F.Cu") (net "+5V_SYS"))
 (segment (start 34.94 60) (end 35.94 57) (width 0.65) (layer "F.Cu") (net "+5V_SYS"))
 (segment (start 43.54 36) (end 43.54 34) (width 0.5) (layer "F.Cu") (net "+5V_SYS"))
 (segment (start 58 84.5) (end 51 84.5) (width 0.24) (layer "F.Cu") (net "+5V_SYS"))
 (segment (start 50.5 89) (end 49.375 94.15) (width 0.24) (layer "F.Cu") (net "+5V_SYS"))
 (segment (start 58 18.16) (end 64.86 18.16) (width 0.65) (layer "F.Cu") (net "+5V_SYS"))
 (via (at 58 36) (size 0.8) (drill 0.4) (layers "F.Cu" "B.Cu") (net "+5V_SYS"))
 (via (at 58 57) (size 0.8) (drill 0.4) (layers "F.Cu" "B.Cu") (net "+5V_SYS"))
 (via (at 58 84.5) (size 0.8) (drill 0.4) (layers "F.Cu" "B.Cu") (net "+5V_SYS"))
 (via (at 58 18.16) (size 0.8) (drill 0.4) (layers "F.Cu" "B.Cu") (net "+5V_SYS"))
 (segment (start 50 119) (end 58 119) (width 0.9) (layer "B.Cu") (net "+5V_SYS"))
 (segment (start 58 119) (end 58 18.16) (width 0.9) (layer "B.Cu") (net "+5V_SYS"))
 (segment (start 52 50) (end 54.0875 50) (width 0.28) (layer "F.Cu") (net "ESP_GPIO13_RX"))
 (segment (start 46.9125 50) (end 52 50) (width 0.28) (layer "F.Cu") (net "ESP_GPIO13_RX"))
 (via (at 52 50) (size 0.8) (drill 0.4) (layers "F.Cu" "B.Cu") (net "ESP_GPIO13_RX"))
 (segment (start 52 15.62) (end 42 15.62) (width 0.28) (layer "B.Cu") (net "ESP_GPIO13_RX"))
 (segment (start 52 50) (end 52 15.62) (width 0.28) (layer "B.Cu") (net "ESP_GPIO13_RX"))
 (segment (start 50 45) (end 46.9125 45) (width 0.28) (layer "F.Cu") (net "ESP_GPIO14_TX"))
 (segment (start 50 43) (end 50 45) (width 0.28) (layer "F.Cu") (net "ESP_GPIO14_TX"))
 (via (at 50 43) (size 0.8) (drill 0.4) (layers "F.Cu" "B.Cu") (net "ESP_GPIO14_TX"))
 (segment (start 39.5 43) (end 50 43) (width 0.28) (layer "B.Cu") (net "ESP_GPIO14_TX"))
 (segment (start 42 20.7) (end 39.5 20.7) (width 0.28) (layer "B.Cu") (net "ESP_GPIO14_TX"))
 (segment (start 39.5 20.7) (end 39.5 43) (width 0.28) (layer "B.Cu") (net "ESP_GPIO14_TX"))
 (segment (start 55.5 94.4) (end 55.625 94.15) (width 0.2) (layer "F.Cu") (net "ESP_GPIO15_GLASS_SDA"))
 (via (at 55.5 94.4) (size 0.8) (drill 0.4) (layers "F.Cu" "B.Cu") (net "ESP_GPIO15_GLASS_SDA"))
 (segment (start 1.2 94.4) (end 55.5 94.4) (width 0.2) (layer "B.Cu") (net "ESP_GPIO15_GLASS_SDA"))
 (segment (start 42 18.16) (end 38.2 18.16) (width 0.2) (layer "B.Cu") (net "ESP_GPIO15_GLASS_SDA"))
 (segment (start 1.2 43) (end 1.2 94.4) (width 0.2) (layer "B.Cu") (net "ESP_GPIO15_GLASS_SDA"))
 (segment (start 38.2 18.16) (end 38.2 43) (width 0.2) (layer "B.Cu") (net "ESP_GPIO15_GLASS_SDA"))
 (segment (start 38.2 43) (end 1.2 43) (width 0.2) (layer "B.Cu") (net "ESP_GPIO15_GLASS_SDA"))
 (segment (start 68.8 93.05) (end 59.375 93.05) (width 0.2) (layer "F.Cu") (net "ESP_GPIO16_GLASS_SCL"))
 (segment (start 59.375 93.05) (end 59.375 94.15) (width 0.2) (layer "F.Cu") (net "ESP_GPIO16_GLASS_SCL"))
 (via (at 68.8 93.05) (size 0.8) (drill 0.4) (layers "F.Cu" "B.Cu") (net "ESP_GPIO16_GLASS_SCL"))
 (segment (start 68.8 10.54) (end 68.8 93.05) (width 0.2) (layer "B.Cu") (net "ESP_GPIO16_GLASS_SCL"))
 (segment (start 64.86 10.54) (end 68.8 10.54) (width 0.2) (layer "B.Cu") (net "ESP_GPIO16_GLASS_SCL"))
 (segment (start 61 28) (end 46.08 28) (width 0.28) (layer "F.Cu") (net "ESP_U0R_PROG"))
 (segment (start 46.08 28) (end 46.08 34) (width 0.28) (layer "F.Cu") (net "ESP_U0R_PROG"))
 (segment (start 61 20.7) (end 61 28) (width 0.28) (layer "F.Cu") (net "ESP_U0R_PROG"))
 (segment (start 64.86 20.7) (end 61 20.7) (width 0.28) (layer "F.Cu") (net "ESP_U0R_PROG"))
 (segment (start 64.86 23.24) (end 63.5 23.24) (width 0.28) (layer "F.Cu") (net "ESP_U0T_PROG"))
 (segment (start 63.5 23.24) (end 63.5 31.5) (width 0.28) (layer "F.Cu") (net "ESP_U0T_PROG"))
 (segment (start 63.5 31.5) (end 48.62 31.5) (width 0.28) (layer "F.Cu") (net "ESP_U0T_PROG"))
 (segment (start 48.62 31.5) (end 48.62 34) (width 0.28) (layer "F.Cu") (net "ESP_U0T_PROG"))
 (segment (start 60.5 39) (end 61 39) (width 0.28) (layer "B.Cu") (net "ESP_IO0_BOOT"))
 (segment (start 60.5 13.08) (end 60.5 39) (width 0.28) (layer "B.Cu") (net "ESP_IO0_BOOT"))
 (segment (start 64.86 13.08) (end 60.5 13.08) (width 0.28) (layer "B.Cu") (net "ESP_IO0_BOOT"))
 (segment (start 41.3 45) (end 45.0875 45) (width 0.28) (layer "F.Cu") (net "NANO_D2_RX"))
 (segment (start 33.4 72) (end 41.3 72) (width 0.28) (layer "F.Cu") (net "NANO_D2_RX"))
 (via (at 41.3 72) (size 0.8) (drill 0.4) (layers "F.Cu" "B.Cu") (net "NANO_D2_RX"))
 (via (at 33.4 72) (size 0.8) (drill 0.4) (layers "F.Cu" "B.Cu") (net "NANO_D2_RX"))
 (via (at 41.3 45) (size 0.8) (drill 0.4) (layers "F.Cu" "B.Cu") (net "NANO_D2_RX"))
 (segment (start 32.4 75.24) (end 33.4 72) (width 0.28) (layer "B.Cu") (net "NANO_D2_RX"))
 (segment (start 41.3 72) (end 41.3 45) (width 0.28) (layer "B.Cu") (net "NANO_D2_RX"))
 (segment (start 38.75 50) (end 45.0875 50) (width 0.28) (layer "F.Cu") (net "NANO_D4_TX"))
 (via (at 38.75 50) (size 0.8) (drill 0.4) (layers "F.Cu" "B.Cu") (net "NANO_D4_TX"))
 (segment (start 28.32 80) (end 38.75 80) (width 0.28) (layer "B.Cu") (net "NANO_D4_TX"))
 (segment (start 38.75 80) (end 38.75 50) (width 0.28) (layer "B.Cu") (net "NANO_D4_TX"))
 (segment (start 27.32 75.24) (end 28.32 80) (width 0.28) (layer "B.Cu") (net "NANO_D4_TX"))
 (segment (start 55 82) (end 61.0875 82) (width 0.24) (layer "F.Cu") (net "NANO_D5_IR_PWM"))
 (via (at 55 82) (size 0.8) (drill 0.4) (layers "F.Cu" "B.Cu") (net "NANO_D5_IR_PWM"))
 (segment (start 24.78 75.24) (end 24.78 82) (width 0.28) (layer "B.Cu") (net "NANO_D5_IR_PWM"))
 (segment (start 24.78 82) (end 55 82) (width 0.28) (layer "B.Cu") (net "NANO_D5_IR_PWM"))
 (segment (start 36 84) (end 37.0875 82) (width 0.24) (layer "F.Cu") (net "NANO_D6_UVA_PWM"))
 (via (at 36 84) (size 0.8) (drill 0.4) (layers "F.Cu" "B.Cu") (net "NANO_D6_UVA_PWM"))
 (segment (start 22.24 84) (end 36 84) (width 0.28) (layer "B.Cu") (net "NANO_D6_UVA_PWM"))
 (segment (start 22.24 75.24) (end 22.24 84) (width 0.28) (layer "B.Cu") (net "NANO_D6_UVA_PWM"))
 (segment (start 48 86) (end 49.0875 80) (width 0.28) (layer "F.Cu") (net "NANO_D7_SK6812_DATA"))
 (via (at 48 86) (size 0.8) (drill 0.4) (layers "F.Cu" "B.Cu") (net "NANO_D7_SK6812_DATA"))
 (segment (start 19.7 86) (end 48 86) (width 0.28) (layer "B.Cu") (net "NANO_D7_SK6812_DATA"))
 (segment (start 19.7 75.24) (end 19.7 86) (width 0.28) (layer "B.Cu") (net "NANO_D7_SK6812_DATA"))
 (segment (start 62.9125 82) (end 63 86.2) (width 0.24) (layer "F.Cu") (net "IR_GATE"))
 (segment (start 66.8 91.95) (end 63.9375 91.95) (width 0.24) (layer "F.Cu") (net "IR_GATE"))
 (segment (start 66.8 86.2) (end 66.8 91.95) (width 0.24) (layer "F.Cu") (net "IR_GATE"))
 (segment (start 62.9125 85) (end 63 86.2) (width 0.24) (layer "F.Cu") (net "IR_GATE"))
 (segment (start 63 86.2) (end 66.8 86.2) (width 0.24) (layer "F.Cu") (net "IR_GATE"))
 (segment (start 45.06 86.2) (end 45.0625 90.05) (width 0.24) (layer "F.Cu") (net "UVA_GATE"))
 (segment (start 38.9125 82) (end 40 86.2) (width 0.24) (layer "F.Cu") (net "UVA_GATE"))
 (segment (start 38.9125 85) (end 40 86.2) (width 0.24) (layer "F.Cu") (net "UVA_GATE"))
 (segment (start 40 86.2) (end 45.06 86.2) (width 0.24) (layer "F.Cu") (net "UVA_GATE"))
 (segment (start 57.5 91) (end 58.125 94.15) (width 0.24) (layer "F.Cu") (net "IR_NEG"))
 (segment (start 62.0625 91) (end 57.5 91) (width 0.24) (layer "F.Cu") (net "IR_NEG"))
 (segment (start 46.9375 91) (end 48.5 91) (width 0.24) (layer "F.Cu") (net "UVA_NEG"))
 (segment (start 48.5 91) (end 46.875 94.15) (width 0.24) (layer "F.Cu") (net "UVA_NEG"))
 (segment (start 58 87.4125) (end 56.5 88) (width 0.24) (layer "F.Cu") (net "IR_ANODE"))
 (segment (start 56.5 88) (end 56.875 94.15) (width 0.24) (layer "F.Cu") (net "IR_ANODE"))
 (segment (start 49.5 89.5) (end 48.125 94.15) (width 0.24) (layer "F.Cu") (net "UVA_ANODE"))
 (segment (start 50 87.4125) (end 49.5 89.5) (width 0.24) (layer "F.Cu") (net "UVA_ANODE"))
 (segment (start 54.5 93.6) (end 54.375 94.15) (width 0.2) (layer "F.Cu") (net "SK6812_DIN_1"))
 (segment (start 50.9125 80) (end 52 80) (width 0.2) (layer "F.Cu") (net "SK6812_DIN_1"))
 (via (at 52 80) (size 0.8) (drill 0.4) (layers "F.Cu" "B.Cu") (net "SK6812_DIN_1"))
 (via (at 54.5 93.6) (size 0.8) (drill 0.4) (layers "F.Cu" "B.Cu") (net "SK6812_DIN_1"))
 (segment (start 56.5 80) (end 56.5 86) (width 0.2) (layer "B.Cu") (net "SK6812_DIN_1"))
 (segment (start 52 80) (end 56.5 80) (width 0.2) (layer "B.Cu") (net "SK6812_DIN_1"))
 (segment (start 54.5 86) (end 54.5 93.6) (width 0.2) (layer "B.Cu") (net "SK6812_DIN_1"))
 (segment (start 56.5 86) (end 54.5 86) (width 0.2) (layer "B.Cu") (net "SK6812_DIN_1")))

